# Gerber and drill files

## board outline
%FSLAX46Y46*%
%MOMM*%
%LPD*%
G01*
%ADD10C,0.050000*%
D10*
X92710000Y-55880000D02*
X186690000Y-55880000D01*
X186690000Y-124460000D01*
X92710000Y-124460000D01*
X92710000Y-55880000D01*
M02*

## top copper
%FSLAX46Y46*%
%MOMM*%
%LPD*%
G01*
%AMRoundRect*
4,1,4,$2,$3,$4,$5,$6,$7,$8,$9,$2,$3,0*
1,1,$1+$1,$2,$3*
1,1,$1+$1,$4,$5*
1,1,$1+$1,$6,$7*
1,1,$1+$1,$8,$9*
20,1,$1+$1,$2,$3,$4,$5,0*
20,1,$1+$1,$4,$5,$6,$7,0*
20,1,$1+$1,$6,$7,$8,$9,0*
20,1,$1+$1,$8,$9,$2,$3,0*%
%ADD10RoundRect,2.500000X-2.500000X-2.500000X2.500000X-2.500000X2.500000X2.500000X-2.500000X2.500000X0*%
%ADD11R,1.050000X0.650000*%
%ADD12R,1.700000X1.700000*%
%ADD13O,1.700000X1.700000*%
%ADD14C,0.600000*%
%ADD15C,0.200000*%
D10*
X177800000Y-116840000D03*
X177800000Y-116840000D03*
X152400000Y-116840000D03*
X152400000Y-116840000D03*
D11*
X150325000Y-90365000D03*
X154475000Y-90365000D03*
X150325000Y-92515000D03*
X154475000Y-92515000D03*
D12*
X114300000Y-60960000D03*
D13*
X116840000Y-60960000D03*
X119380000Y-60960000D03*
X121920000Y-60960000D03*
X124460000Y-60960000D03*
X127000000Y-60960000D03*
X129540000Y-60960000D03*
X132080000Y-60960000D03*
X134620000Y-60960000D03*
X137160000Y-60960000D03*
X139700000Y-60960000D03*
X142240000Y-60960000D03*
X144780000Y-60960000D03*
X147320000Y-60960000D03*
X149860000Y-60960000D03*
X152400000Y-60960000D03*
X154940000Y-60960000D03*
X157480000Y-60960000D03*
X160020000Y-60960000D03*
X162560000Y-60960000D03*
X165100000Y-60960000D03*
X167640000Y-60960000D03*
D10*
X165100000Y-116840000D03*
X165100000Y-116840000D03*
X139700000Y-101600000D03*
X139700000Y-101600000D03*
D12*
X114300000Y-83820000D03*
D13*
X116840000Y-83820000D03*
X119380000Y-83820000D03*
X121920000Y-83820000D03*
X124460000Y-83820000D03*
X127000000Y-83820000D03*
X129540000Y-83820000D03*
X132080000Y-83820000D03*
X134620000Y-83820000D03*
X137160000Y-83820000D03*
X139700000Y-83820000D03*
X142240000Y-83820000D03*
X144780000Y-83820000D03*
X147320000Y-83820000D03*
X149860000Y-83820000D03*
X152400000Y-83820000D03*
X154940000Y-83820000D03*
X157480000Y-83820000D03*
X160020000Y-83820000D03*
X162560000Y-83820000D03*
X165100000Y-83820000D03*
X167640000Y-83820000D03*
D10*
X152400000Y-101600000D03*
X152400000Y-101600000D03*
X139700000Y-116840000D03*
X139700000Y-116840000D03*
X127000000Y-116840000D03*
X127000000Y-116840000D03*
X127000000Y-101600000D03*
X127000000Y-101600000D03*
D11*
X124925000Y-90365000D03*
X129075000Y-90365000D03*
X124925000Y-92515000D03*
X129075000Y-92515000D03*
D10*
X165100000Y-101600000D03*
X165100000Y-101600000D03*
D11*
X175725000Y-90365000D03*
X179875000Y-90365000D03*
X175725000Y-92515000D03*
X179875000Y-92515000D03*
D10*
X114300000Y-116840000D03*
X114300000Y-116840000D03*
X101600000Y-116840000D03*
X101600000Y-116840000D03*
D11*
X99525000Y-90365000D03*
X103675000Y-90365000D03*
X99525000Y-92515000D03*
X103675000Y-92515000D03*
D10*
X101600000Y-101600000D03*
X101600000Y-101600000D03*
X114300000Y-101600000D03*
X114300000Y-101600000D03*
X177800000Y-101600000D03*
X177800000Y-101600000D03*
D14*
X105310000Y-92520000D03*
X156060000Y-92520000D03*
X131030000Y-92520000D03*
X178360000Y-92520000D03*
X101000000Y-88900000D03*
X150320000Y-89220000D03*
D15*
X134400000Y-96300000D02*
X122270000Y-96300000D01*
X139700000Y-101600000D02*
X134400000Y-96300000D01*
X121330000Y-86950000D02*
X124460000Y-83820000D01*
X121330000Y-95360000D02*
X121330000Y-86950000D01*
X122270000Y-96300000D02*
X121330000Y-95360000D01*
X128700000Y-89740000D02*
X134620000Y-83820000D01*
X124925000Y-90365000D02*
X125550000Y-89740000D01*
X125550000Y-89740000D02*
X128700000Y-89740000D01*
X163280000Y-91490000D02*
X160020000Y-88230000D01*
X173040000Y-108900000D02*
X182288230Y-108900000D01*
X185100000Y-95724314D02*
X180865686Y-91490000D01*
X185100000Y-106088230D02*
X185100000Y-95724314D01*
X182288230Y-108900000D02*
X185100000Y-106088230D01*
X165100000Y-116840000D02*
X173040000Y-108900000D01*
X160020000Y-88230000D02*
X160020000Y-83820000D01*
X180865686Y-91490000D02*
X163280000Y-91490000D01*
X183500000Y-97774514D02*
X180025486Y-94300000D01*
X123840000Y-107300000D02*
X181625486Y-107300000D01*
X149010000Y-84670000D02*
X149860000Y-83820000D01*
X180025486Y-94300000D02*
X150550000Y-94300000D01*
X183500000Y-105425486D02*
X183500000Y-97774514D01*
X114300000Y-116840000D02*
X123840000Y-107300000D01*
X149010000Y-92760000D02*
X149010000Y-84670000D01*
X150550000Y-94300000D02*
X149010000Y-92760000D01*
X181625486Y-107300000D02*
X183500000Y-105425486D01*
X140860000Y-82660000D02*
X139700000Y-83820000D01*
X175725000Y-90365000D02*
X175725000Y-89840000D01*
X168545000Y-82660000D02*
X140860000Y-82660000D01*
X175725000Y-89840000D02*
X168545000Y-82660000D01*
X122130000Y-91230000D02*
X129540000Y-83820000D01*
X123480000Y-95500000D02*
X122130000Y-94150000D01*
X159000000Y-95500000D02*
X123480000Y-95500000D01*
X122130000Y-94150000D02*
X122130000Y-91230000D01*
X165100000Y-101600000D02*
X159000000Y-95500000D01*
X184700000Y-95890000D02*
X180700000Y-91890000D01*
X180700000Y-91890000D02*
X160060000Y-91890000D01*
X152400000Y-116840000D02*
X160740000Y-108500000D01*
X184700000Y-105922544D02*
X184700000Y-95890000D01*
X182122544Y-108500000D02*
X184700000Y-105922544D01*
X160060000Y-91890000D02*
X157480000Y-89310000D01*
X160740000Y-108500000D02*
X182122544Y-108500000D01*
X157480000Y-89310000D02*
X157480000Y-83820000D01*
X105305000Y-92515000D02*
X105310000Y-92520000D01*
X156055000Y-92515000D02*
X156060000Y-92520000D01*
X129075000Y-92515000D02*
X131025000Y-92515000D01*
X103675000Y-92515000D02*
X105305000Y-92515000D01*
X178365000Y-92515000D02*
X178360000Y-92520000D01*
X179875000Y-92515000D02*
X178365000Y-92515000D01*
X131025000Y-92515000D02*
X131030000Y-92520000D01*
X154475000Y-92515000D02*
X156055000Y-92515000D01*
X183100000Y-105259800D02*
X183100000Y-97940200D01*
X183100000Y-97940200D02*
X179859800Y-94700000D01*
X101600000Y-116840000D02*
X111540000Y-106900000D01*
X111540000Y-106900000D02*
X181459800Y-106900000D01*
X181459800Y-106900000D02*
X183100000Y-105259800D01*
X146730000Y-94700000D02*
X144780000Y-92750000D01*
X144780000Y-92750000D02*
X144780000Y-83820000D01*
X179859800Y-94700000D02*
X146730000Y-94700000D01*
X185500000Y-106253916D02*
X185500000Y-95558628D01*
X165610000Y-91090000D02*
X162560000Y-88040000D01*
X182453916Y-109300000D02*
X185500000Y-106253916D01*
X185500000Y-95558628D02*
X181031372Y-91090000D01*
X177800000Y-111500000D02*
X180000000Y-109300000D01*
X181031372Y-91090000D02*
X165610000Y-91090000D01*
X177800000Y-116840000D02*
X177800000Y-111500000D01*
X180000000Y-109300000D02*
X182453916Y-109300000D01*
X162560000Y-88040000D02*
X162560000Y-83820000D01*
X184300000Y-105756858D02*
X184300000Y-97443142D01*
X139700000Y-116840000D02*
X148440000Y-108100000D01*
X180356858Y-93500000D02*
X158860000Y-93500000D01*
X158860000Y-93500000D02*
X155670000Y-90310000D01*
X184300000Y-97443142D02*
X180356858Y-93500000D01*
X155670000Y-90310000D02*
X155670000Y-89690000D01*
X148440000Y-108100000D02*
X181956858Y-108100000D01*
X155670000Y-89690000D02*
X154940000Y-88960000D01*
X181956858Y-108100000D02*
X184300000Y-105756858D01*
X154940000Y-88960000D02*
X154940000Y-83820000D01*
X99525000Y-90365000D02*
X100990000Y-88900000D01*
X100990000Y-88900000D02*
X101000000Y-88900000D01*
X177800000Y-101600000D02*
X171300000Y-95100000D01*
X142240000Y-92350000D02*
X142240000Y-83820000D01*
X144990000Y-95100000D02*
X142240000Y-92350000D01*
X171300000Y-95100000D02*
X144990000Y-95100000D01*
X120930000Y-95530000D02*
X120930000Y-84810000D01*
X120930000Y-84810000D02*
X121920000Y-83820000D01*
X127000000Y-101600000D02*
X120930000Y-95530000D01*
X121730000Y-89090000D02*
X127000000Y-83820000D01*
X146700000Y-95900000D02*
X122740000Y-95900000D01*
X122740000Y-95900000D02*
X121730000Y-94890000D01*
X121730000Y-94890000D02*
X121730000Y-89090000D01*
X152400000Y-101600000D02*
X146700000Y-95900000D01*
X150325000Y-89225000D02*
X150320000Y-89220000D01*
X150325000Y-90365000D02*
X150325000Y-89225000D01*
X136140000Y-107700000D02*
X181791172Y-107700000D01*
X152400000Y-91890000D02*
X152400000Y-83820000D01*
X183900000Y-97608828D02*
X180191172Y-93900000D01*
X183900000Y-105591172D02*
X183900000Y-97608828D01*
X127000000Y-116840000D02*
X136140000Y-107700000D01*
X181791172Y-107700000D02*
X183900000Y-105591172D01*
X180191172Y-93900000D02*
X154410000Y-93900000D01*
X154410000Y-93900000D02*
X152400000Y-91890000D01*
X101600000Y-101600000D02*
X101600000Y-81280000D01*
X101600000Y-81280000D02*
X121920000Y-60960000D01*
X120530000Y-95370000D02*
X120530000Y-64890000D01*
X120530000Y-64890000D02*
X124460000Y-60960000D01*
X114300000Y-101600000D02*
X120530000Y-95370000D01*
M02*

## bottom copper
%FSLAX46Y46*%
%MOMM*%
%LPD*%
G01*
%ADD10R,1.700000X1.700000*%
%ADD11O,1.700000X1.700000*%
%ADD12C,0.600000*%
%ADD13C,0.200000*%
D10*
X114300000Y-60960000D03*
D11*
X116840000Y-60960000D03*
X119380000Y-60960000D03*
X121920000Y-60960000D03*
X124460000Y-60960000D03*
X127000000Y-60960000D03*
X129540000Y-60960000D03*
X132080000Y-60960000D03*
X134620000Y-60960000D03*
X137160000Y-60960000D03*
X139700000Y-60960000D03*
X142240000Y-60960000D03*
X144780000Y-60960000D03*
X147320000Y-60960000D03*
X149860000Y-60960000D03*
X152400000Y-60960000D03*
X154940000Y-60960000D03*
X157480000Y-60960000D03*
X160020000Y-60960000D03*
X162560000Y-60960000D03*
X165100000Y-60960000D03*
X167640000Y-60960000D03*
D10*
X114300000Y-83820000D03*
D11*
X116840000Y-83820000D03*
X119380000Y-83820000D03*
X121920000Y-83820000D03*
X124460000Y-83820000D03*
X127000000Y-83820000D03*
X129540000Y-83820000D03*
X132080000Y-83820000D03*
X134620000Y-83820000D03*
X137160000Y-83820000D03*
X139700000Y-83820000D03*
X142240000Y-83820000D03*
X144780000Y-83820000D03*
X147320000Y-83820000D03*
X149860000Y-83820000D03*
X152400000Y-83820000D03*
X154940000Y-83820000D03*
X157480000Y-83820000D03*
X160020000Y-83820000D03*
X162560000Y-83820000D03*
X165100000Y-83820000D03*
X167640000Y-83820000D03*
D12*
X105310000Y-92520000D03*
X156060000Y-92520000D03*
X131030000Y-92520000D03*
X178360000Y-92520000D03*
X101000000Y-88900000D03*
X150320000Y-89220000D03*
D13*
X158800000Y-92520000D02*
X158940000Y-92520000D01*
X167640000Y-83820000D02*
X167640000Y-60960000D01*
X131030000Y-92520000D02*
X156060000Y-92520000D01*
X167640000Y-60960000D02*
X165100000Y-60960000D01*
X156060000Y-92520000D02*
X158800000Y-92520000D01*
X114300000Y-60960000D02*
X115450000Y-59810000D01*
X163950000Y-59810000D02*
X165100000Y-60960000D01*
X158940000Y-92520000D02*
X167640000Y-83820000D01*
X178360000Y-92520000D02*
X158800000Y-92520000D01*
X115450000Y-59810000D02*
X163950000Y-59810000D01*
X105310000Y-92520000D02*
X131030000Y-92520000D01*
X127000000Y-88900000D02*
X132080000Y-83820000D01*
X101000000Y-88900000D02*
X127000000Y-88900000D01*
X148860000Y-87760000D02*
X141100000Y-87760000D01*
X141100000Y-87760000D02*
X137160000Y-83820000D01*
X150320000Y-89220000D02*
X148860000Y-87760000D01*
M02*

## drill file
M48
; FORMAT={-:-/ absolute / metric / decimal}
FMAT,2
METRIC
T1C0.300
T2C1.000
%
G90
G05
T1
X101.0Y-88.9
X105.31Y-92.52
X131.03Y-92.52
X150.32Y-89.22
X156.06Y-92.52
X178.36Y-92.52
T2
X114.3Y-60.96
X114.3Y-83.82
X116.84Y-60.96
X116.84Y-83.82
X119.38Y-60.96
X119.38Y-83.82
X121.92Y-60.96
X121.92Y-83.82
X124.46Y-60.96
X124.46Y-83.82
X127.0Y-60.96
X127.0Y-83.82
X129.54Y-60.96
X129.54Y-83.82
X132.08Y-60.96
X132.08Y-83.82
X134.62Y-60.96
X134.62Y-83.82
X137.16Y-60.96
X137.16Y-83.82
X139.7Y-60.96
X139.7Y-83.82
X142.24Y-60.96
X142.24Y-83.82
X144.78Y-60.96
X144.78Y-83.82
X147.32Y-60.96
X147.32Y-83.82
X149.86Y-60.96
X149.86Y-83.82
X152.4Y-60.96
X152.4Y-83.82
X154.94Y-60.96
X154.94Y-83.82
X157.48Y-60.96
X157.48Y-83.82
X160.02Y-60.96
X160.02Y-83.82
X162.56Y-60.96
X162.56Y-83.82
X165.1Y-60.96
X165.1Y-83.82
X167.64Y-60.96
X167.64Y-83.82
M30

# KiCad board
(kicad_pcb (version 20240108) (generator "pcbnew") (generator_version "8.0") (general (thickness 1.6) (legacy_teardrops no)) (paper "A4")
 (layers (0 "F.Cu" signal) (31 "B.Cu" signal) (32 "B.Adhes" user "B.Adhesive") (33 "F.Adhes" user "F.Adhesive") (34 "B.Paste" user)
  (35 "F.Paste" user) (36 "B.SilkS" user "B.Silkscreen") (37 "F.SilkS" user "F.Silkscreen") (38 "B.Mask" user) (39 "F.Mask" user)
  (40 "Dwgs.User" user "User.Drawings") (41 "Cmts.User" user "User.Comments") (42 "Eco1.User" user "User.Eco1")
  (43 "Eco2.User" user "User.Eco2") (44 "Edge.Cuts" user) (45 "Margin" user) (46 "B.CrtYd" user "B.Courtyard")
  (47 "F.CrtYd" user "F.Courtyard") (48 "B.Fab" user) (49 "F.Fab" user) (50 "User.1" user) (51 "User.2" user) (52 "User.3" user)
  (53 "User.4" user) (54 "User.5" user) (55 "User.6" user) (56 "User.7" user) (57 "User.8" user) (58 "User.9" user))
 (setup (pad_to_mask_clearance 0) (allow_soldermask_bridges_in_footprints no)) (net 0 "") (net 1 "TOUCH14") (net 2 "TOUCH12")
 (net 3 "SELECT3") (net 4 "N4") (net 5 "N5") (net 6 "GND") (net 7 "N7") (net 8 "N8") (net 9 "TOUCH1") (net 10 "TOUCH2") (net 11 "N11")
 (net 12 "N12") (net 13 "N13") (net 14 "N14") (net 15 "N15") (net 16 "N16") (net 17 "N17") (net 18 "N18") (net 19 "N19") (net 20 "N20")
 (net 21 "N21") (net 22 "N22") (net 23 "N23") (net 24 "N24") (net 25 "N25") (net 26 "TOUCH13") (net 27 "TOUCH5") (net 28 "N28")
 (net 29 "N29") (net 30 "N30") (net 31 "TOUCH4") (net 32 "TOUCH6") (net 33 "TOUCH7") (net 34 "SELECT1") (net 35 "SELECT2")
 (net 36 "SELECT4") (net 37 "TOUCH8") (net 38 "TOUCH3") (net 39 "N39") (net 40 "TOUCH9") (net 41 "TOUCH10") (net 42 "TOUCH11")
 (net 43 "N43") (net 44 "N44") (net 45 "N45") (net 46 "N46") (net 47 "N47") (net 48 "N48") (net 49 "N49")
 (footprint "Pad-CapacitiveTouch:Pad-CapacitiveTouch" (layer "F.Cu") (at 177.8 116.84)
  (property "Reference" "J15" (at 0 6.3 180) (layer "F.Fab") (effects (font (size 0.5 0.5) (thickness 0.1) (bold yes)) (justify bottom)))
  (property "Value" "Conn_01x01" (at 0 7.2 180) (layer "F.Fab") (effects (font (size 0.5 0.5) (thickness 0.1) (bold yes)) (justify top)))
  (pad "1" smd roundrect (at 0 0) (size 10 10) (layers "F.Cu") (roundrect_rratio 0.25) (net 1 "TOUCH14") (thermal_bridge_angle 0))
  (pad "1" smd roundrect (at 0 0) (size 10 10) (layers "F.Cu" "F.Mask") (roundrect_rratio 0.25) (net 1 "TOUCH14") (thermal_bridge_angle 0)))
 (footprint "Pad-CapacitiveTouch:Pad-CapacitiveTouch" (layer "F.Cu") (at 152.4 116.84)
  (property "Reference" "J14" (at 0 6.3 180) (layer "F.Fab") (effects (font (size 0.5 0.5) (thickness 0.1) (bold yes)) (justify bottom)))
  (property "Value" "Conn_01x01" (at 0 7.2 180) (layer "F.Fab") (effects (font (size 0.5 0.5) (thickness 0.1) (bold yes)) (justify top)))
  (pad "1" smd roundrect (at 0 0) (size 10 10) (layers "F.Cu") (roundrect_rratio 0.25) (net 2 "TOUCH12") (thermal_bridge_angle 0))
  (pad "1" smd roundrect (at 0 0) (size 10 10) (layers "F.Cu" "F.Mask") (roundrect_rratio 0.25) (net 2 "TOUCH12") (thermal_bridge_angle 0)))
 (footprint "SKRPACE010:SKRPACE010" (layer "F.Cu") (at 152.4 91.44)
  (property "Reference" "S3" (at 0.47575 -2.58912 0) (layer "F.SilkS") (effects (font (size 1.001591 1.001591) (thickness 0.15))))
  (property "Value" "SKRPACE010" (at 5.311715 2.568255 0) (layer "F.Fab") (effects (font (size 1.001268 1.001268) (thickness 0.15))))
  (pad "1" smd rect (at -2.075 -1.075) (size 1.05 0.65) (layers "F.Cu" "F.Paste" "F.Mask") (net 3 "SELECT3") (solder_mask_margin 0.102))
  (pad "2" smd rect (at 2.075 -1.075) (size 1.05 0.65) (layers "F.Cu" "F.Paste" "F.Mask") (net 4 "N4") (solder_mask_margin 0.102))
  (pad "3" smd rect (at -2.075 1.075) (size 1.05 0.65) (layers "F.Cu" "F.Paste" "F.Mask") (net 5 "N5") (solder_mask_margin 0.102))
  (pad "4" smd rect (at 2.075 1.075) (size 1.05 0.65) (layers "F.Cu" "F.Paste" "F.Mask") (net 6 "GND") (solder_mask_margin 0.102)))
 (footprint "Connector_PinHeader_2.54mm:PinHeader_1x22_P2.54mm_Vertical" (layer "F.Cu") (at 114.3 60.96 90)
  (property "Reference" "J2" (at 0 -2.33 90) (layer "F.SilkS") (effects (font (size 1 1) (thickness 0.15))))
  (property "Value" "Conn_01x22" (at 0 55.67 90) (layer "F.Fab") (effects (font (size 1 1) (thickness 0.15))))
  (pad "1" thru_hole rect (at 0 0 90) (size 1.7 1.7) (drill 1) (layers "*.Cu" "*.Mask") (remove_unused_layers no) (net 6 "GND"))
  (pad "2" thru_hole oval (at 0 2.54 90) (size 1.7 1.7) (drill 1) (layers "*.Cu" "*.Mask") (remove_unused_layers no) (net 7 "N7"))
  (pad "3" thru_hole oval (at 0 5.08 90) (size 1.7 1.7) (drill 1) (layers "*.Cu" "*.Mask") (remove_unused_layers no) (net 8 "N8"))
  (pad "4" thru_hole oval (at 0 7.62 90) (size 1.7 1.7) (drill 1) (layers "*.Cu" "*.Mask") (remove_unused_layers no) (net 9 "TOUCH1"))
  (pad "5" thru_hole oval (at 0 10.16 90) (size 1.7 1.7) (drill 1) (layers "*.Cu" "*.Mask") (remove_unused_layers no) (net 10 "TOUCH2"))
  (pad "6" thru_hole oval (at 0 12.7 90) (size 1.7 1.7) (drill 1) (layers "*.Cu" "*.Mask") (remove_unused_layers no) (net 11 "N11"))
  (pad "7" thru_hole oval (at 0 15.24 90) (size 1.7 1.7) (drill 1) (layers "*.Cu" "*.Mask") (remove_unused_layers no) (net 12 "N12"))
  (pad "8" thru_hole oval (at 0 17.78 90) (size 1.7 1.7) (drill 1) (layers "*.Cu" "*.Mask") (remove_unused_layers no) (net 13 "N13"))
  (pad "9" thru_hole oval (at 0 20.32 90) (size 1.7 1.7) (drill 1) (layers "*.Cu" "*.Mask") (remove_unused_layers no) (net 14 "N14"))
  (pad "10" thru_hole oval (at 0 22.86 90) (size 1.7 1.7) (drill 1) (layers "*.Cu" "*.Mask") (remove_unused_layers no) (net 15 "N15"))
  (pad "11" thru_hole oval (at 0 25.4 90) (size 1.7 1.7) (drill 1) (layers "*.Cu" "*.Mask") (remove_unused_layers no) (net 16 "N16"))
  (pad "12" thru_hole oval (at 0 27.94 90) (size 1.7 1.7) (drill 1) (layers "*.Cu" "*.Mask") (remove_unused_layers no) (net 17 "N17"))
  (pad "13" thru_hole oval (at 0 30.48 90) (size 1.7 1.7) (drill 1) (layers "*.Cu" "*.Mask") (remove_unused_layers no) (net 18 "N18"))
  (pad "14" thru_hole oval (at 0 33.02 90) (size 1.7 1.7) (drill 1) (layers "*.Cu" "*.Mask") (remove_unused_layers no) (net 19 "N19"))
  (pad "15" thru_hole oval (at 0 35.56 90) (size 1.7 1.7) (drill 1) (layers "*.Cu" "*.Mask") (remove_unused_layers no) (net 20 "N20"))
  (pad "16" thru_hole oval (at 0 38.1 90) (size 1.7 1.7) (drill 1) (layers "*.Cu" "*.Mask") (remove_unused_layers no) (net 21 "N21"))
  (pad "17" thru_hole oval (at 0 40.64 90) (size 1.7 1.7) (drill 1) (layers "*.Cu" "*.Mask") (remove_unused_layers no) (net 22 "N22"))
  (pad "18" thru_hole oval (at 0 43.18 90) (size 1.7 1.7) (drill 1) (layers "*.Cu" "*.Mask") (remove_unused_layers no) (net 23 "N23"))
  (pad "19" thru_hole oval (at 0 45.72 90) (size 1.7 1.7) (drill 1) (layers "*.Cu" "*.Mask") (remove_unused_layers no) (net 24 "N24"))
  (pad "20" thru_hole oval (at 0 48.26 90) (size 1.7 1.7) (drill 1) (layers "*.Cu" "*.Mask") (remove_unused_layers no) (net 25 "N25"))
  (pad "21" thru_hole oval (at 0 50.8 90) (size 1.7 1.7) (drill 1) (layers "*.Cu" "*.Mask") (remove_unused_layers no) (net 6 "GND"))
  (pad "22" thru_hole oval (at 0 53.34 90) (size 1.7 1.7) (drill 1) (layers "*.Cu" "*.Mask") (remove_unused_layers no) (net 6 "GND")))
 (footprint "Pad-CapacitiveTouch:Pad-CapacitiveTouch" (layer "F.Cu") (at 165.1 116.84)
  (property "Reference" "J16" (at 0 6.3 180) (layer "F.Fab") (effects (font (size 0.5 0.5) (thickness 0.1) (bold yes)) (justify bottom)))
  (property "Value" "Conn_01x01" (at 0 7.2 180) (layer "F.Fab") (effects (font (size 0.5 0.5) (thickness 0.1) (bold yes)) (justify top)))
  (pad "1" smd roundrect (at 0 0) (size 10 10) (layers "F.Cu") (roundrect_rratio 0.25) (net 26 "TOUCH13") (thermal_bridge_angle 0))
  (pad "1" smd roundrect (at 0 0) (size 10 10) (layers "F.Cu" "F.Mask") (roundrect_rratio 0.25) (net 26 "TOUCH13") (thermal_bridge_angle 0)))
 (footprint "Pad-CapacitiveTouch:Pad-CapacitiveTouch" (layer "F.Cu") (at 139.7 101.6)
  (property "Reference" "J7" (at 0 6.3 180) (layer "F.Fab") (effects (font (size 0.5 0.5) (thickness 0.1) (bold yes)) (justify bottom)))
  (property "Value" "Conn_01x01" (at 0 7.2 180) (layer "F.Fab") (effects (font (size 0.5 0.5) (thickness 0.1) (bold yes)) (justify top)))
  (pad "1" smd roundrect (at 0 0) (size 10 10) (layers "F.Cu") (roundrect_rratio 0.25) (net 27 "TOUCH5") (thermal_bridge_angle 0))
  (pad "1" smd roundrect (at 0 0) (size 10 10) (layers "F.Cu" "F.Mask") (roundrect_rratio 0.25) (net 27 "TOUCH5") (thermal_bridge_angle 0)))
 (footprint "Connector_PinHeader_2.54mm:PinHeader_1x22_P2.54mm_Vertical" (layer "F.Cu") (at 114.3 83.82 90)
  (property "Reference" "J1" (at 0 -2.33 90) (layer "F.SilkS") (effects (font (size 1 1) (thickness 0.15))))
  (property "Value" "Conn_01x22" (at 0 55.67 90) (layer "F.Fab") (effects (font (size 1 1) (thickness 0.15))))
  (pad "1" thru_hole rect (at 0 0 90) (size 1.7 1.7) (drill 1) (layers "*.Cu" "*.Mask") (remove_unused_layers no) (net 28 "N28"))
  (pad "2" thru_hole oval (at 0 2.54 90) (size 1.7 1.7) (drill 1) (layers "*.Cu" "*.Mask") (remove_unused_layers no) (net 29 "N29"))
  (pad "3" thru_hole oval (at 0 5.08 90) (size 1.7 1.7) (drill 1) (layers "*.Cu" "*.Mask") (remove_unused_layers no) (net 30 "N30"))
  (pad "4" thru_hole oval (at 0 7.62 90) (size 1.7 1.7) (drill 1) (layers "*.Cu" "*.Mask") (remove_unused_layers no) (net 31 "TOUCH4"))
  (pad "5" thru_hole oval (at 0 10.16 90) (size 1.7 1.7) (drill 1) (layers "*.Cu" "*.Mask") (remove_unused_layers no) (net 27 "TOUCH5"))
  (pad "6" thru_hole oval (at 0 12.7 90) (size 1.7 1.7) (drill 1) (layers "*.Cu" "*.Mask") (remove_unused_layers no) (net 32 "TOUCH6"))
  (pad "7" thru_hole oval (at 0 15.24 90) (size 1.7 1.7) (drill 1) (layers "*.Cu" "*.Mask") (remove_unused_layers no) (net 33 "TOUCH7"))
  (pad "8" thru_hole oval (at 0 17.78 90) (size 1.7 1.7) (drill 1) (layers "*.Cu" "*.Mask") (remove_unused_layers no) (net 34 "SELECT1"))
  (pad "9" thru_hole oval (at 0 20.32 90) (size 1.7 1.7) (drill 1) (layers "*.Cu" "*.Mask") (remove_unused_layers no) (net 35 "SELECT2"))
  (pad "10" thru_hole oval (at 0 22.86 90) (size 1.7 1.7) (drill 1) (layers "*.Cu" "*.Mask") (remove_unused_layers no) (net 3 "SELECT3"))
  (pad "11" thru_hole oval (at 0 25.4 90) (size 1.7 1.7) (drill 1) (layers "*.Cu" "*.Mask") (remove_unused_layers no) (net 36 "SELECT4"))
  (pad "12" thru_hole oval (at 0 27.94 90) (size 1.7 1.7) (drill 1) (layers "*.Cu" "*.Mask") (remove_unused_layers no) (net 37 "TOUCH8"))
  (pad "13" thru_hole oval (at 0 30.48 90) (size 1.7 1.7) (drill 1) (layers "*.Cu" "*.Mask") (remove_unused_layers no) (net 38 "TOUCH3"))
  (pad "14" thru_hole oval (at 0 33.02 90) (size 1.7 1.7) (drill 1) (layers "*.Cu" "*.Mask") (remove_unused_layers no) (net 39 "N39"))
  (pad "15" thru_hole oval (at 0 35.56 90) (size 1.7 1.7) (drill 1) (layers "*.Cu" "*.Mask") (remove_unused_layers no) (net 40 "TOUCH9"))
  (pad "16" thru_hole oval (at 0 38.1 90) (size 1.7 1.7) (drill 1) (layers "*.Cu" "*.Mask") (remove_unused_layers no) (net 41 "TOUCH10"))
  (pad "17" thru_hole oval (at 0 40.64 90) (size 1.7 1.7) (drill 1) (layers "*.Cu" "*.Mask") (remove_unused_layers no) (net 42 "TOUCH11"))
  (pad "18" thru_hole oval (at 0 43.18 90) (size 1.7 1.7) (drill 1) (layers "*.Cu" "*.Mask") (remove_unused_layers no) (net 2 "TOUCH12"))
  (pad "19" thru_hole oval (at 0 45.72 90) (size 1.7 1.7) (drill 1) (layers "*.Cu" "*.Mask") (remove_unused_layers no) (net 26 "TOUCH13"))
  (pad "20" thru_hole oval (at 0 48.26 90) (size 1.7 1.7) (drill 1) (layers "*.Cu" "*.Mask") (remove_unused_layers no) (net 1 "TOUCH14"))
  (pad "21" thru_hole oval (at 0 50.8 90) (size 1.7 1.7) (drill 1) (layers "*.Cu" "*.Mask") (remove_unused_layers no) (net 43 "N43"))
  (pad "22" thru_hole oval (at 0 53.34 90) (size 1.7 1.7) (drill 1) (layers "*.Cu" "*.Mask") (remove_unused_layers no) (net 6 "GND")))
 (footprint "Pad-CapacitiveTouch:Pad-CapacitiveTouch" (layer "F.Cu") (at 152.4 101.6)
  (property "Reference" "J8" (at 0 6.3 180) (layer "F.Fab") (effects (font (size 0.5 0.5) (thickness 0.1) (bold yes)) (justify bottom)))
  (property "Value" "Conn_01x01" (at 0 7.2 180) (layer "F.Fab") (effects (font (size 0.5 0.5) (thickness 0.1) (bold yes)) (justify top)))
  (pad "1" smd roundrect (at 0 0) (size 10 10) (layers "F.Cu") (roundrect_rratio 0.25) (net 32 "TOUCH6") (thermal_bridge_angle 0))
  (pad "1" smd roundrect (at 0 0) (size 10 10) (layers "F.Cu" "F.Mask") (roundrect_rratio 0.25) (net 32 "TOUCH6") (thermal_bridge_angle 0)))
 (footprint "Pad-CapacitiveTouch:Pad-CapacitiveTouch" (layer "F.Cu") (at 139.7 116.84)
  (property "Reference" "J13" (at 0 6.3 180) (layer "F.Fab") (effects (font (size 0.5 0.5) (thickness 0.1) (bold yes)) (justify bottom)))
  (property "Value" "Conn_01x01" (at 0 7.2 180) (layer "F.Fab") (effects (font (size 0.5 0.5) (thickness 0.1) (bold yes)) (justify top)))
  (pad "1" smd roundrect (at 0 0) (size 10 10) (layers "F.Cu") (roundrect_rratio 0.25) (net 42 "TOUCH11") (thermal_bridge_angle 0))
  (pad "1" smd roundrect (at 0 0) (size 10 10) (layers "F.Cu" "F.Mask") (roundrect_rratio 0.25) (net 42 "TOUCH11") (thermal_bridge_angle 0)))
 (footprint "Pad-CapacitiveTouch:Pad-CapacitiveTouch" (layer "F.Cu") (at 127 116.84)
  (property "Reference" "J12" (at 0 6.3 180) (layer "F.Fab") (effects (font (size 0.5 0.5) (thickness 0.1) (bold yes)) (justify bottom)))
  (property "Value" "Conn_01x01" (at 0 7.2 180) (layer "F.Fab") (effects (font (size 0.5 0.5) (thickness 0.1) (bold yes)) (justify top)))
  (pad "1" smd roundrect (at 0 0) (size 10 10) (layers "F.Cu") (roundrect_rratio 0.25) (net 41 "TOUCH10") (thermal_bridge_angle 0))
  (pad "1" smd roundrect (at 0 0) (size 10 10) (layers "F.Cu" "F.Mask") (roundrect_rratio 0.25) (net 41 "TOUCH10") (thermal_bridge_angle 0)))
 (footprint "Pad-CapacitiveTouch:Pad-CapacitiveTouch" (layer "F.Cu") (at 127 101.6)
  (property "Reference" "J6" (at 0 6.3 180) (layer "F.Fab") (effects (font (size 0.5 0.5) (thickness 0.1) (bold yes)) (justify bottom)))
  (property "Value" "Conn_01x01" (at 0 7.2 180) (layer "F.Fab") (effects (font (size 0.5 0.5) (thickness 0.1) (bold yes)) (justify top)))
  (pad "1" smd roundrect (at 0 0) (size 10 10) (layers "F.Cu") (roundrect_rratio 0.25) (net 31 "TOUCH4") (thermal_bridge_angle 0))
  (pad "1" smd roundrect (at 0 0) (size 10 10) (layers "F.Cu" "F.Mask") (roundrect_rratio 0.25) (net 31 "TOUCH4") (thermal_bridge_angle 0)))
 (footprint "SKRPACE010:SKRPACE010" (layer "F.Cu") (at 127 91.44)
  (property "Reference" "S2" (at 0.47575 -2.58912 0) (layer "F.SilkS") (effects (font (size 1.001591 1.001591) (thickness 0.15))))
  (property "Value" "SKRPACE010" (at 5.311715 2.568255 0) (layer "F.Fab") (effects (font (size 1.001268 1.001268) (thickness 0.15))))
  (pad "1" smd rect (at -2.075 -1.075) (size 1.05 0.65) (layers "F.Cu" "F.Paste" "F.Mask") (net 35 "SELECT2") (solder_mask_margin 0.102))
  (pad "2" smd rect (at 2.075 -1.075) (size 1.05 0.65) (layers "F.Cu" "F.Paste" "F.Mask") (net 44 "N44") (solder_mask_margin 0.102))
  (pad "3" smd rect (at -2.075 1.075) (size 1.05 0.65) (layers "F.Cu" "F.Paste" "F.Mask") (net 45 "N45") (solder_mask_margin 0.102))
  (pad "4" smd rect (at 2.075 1.075) (size 1.05 0.65) (layers "F.Cu" "F.Paste" "F.Mask") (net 6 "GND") (solder_mask_margin 0.102)))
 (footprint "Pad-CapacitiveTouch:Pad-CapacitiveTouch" (layer "F.Cu") (at 165.1 101.6)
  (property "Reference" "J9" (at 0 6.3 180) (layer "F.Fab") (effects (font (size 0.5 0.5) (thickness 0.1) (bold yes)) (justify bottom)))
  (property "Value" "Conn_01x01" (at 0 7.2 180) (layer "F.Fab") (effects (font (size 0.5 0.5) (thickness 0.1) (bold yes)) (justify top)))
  (pad "1" smd roundrect (at 0 0) (size 10 10) (layers "F.Cu") (roundrect_rratio 0.25) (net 33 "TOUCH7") (thermal_bridge_angle 0))
  (pad "1" smd roundrect (at 0 0) (size 10 10) (layers "F.Cu" "F.Mask") (roundrect_rratio 0.25) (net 33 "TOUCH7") (thermal_bridge_angle 0)))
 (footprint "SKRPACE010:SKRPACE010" (layer "F.Cu") (at 177.8 91.44)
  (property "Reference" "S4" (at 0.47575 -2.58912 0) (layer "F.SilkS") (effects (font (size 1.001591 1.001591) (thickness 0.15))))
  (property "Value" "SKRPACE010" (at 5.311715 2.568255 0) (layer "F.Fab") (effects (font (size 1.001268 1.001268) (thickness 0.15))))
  (pad "1" smd rect (at -2.075 -1.075) (size 1.05 0.65) (layers "F.Cu" "F.Paste" "F.Mask") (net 36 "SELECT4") (solder_mask_margin 0.102))
  (pad "2" smd rect (at 2.075 -1.075) (size 1.05 0.65) (layers "F.Cu" "F.Paste" "F.Mask") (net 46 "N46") (solder_mask_margin 0.102))
  (pad "3" smd rect (at -2.075 1.075) (size 1.05 0.65) (layers "F.Cu" "F.Paste" "F.Mask") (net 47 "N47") (solder_mask_margin 0.102))
  (pad "4" smd rect (at 2.075 1.075) (size 1.05 0.65) (layers "F.Cu" "F.Paste" "F.Mask") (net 6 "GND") (solder_mask_margin 0.102)))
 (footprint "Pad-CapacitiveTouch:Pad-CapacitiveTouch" (layer "F.Cu") (at 114.3 116.84)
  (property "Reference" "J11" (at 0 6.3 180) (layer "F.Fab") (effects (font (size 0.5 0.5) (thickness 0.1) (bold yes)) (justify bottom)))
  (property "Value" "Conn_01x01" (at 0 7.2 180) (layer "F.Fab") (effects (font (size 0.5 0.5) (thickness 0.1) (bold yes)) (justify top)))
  (pad "1" smd roundrect (at 0 0) (size 10 10) (layers "F.Cu") (roundrect_rratio 0.25) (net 40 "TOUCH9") (thermal_bridge_angle 0))
  (pad "1" smd roundrect (at 0 0) (size 10 10) (layers "F.Cu" "F.Mask") (roundrect_rratio 0.25) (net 40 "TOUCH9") (thermal_bridge_angle 0)))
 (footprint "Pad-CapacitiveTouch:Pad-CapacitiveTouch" (layer "F.Cu") (at 101.6 116.84)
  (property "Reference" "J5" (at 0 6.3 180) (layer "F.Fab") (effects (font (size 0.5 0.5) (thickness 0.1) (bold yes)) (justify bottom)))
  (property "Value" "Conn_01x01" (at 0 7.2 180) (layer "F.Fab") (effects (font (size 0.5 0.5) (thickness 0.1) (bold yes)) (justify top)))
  (pad "1" smd roundrect (at 0 0) (size 10 10) (layers "F.Cu") (roundrect_rratio 0.25) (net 38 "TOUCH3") (thermal_bridge_angle 0))
  (pad "1" smd roundrect (at 0 0) (size 10 10) (layers "F.Cu" "F.Mask") (roundrect_rratio 0.25) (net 38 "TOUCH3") (thermal_bridge_angle 0)))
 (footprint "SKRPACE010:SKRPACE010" (layer "F.Cu") (at 101.6 91.44)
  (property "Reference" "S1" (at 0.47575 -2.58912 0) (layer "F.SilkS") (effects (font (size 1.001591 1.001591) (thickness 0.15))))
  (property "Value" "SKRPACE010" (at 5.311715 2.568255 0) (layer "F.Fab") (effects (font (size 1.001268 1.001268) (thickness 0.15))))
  (pad "1" smd rect (at -2.075 -1.075) (size 1.05 0.65) (layers "F.Cu" "F.Paste" "F.Mask") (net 34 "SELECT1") (solder_mask_margin 0.102))
  (pad "2" smd rect (at 2.075 -1.075) (size 1.05 0.65) (layers "F.Cu" "F.Paste" "F.Mask") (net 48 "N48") (solder_mask_margin 0.102))
  (pad "3" smd rect (at -2.075 1.075) (size 1.05 0.65) (layers "F.Cu" "F.Paste" "F.Mask") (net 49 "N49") (solder_mask_margin 0.102))
  (pad "4" smd rect (at 2.075 1.075) (size 1.05 0.65) (layers "F.Cu" "F.Paste" "F.Mask") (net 6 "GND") (solder_mask_margin 0.102)))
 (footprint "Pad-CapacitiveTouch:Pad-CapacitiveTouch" (layer "F.Cu") (at 101.6 101.6)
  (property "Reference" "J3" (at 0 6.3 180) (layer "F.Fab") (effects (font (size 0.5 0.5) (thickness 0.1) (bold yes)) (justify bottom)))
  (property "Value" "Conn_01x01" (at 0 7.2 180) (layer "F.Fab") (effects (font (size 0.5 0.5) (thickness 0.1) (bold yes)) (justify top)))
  (pad "1" smd roundrect (at 0 0) (size 10 10) (layers "F.Cu") (roundrect_rratio 0.25) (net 9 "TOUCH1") (thermal_bridge_angle 0))
  (pad "1" smd roundrect (at 0 0) (size 10 10) (layers "F.Cu" "F.Mask") (roundrect_rratio 0.25) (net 9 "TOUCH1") (thermal_bridge_angle 0)))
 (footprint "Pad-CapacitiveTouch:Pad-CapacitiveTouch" (layer "F.Cu") (at 114.3 101.6)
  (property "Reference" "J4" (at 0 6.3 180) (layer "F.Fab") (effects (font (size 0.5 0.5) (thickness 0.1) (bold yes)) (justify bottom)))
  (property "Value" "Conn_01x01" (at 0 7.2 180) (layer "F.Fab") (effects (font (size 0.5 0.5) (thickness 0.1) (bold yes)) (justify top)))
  (pad "1" smd roundrect (at 0 0) (size 10 10) (layers "F.Cu") (roundrect_rratio 0.25) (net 10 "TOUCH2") (thermal_bridge_angle 0))
  (pad "1" smd roundrect (at 0 0) (size 10 10) (layers "F.Cu" "F.Mask") (roundrect_rratio 0.25) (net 10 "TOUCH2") (thermal_bridge_angle 0)))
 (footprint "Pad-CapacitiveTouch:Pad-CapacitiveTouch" (layer "F.Cu") (at 177.8 101.6)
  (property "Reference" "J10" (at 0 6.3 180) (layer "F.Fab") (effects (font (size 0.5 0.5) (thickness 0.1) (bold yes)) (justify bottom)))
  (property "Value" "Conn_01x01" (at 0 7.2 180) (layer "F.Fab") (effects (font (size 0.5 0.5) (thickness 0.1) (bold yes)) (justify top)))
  (pad "1" smd roundrect (at 0 0) (size 10 10) (layers "F.Cu") (roundrect_rratio 0.25) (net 37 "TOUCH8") (thermal_bridge_angle 0))
  (pad "1" smd roundrect (at 0 0) (size 10 10) (layers "F.Cu" "F.Mask") (roundrect_rratio 0.25) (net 37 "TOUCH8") (thermal_bridge_angle 0)))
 (gr_rect (start 92.71 55.88) (end 186.69 124.46) (stroke (width 0.05) (type default)) (fill none) (layer "Edge.Cuts"))
 (segment (start 134.4 96.3) (end 122.27 96.3) (width 0.2) (layer "F.Cu") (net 27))
 (segment (start 139.7 101.6) (end 134.4 96.3) (width 0.2) (layer "F.Cu") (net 27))
 (segment (start 121.33 86.95) (end 124.46 83.82) (width 0.2) (layer "F.Cu") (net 27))
 (segment (start 121.33 95.36) (end 121.33 86.95) (width 0.2) (layer "F.Cu") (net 27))
 (segment (start 122.27 96.3) (end 121.33 95.36) (width 0.2) (layer "F.Cu") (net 27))
 (segment (start 128.7 89.74) (end 134.62 83.82) (width 0.2) (layer "F.Cu") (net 35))
 (segment (start 124.925 90.365) (end 125.55 89.74) (width 0.2) (layer "F.Cu") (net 35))
 (segment (start 125.55 89.74) (end 128.7 89.74) (width 0.2) (layer "F.Cu") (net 35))
 (segment (start 163.28 91.49) (end 160.02 88.23) (width 0.2) (layer "F.Cu") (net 26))
 (segment (start 173.04 108.9) (end 182.28823 108.9) (width 0.2) (layer "F.Cu") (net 26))
 (segment (start 185.1 95.724314) (end 180.865686 91.49) (width 0.2) (layer "F.Cu") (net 26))
 (segment (start 185.1 106.08823) (end 185.1 95.724314) (width 0.2) (layer "F.Cu") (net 26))
 (segment (start 182.28823 108.9) (end 185.1 106.08823) (width 0.2) (layer "F.Cu") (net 26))
 (segment (start 165.1 116.84) (end 173.04 108.9) (width 0.2) (layer "F.Cu") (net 26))
 (segment (start 160.02 88.23) (end 160.02 83.82) (width 0.2) (layer "F.Cu") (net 26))
 (segment (start 180.865686 91.49) (end 163.28 91.49) (width 0.2) (layer "F.Cu") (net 26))
 (segment (start 183.5 97.774514) (end 180.025486 94.3) (width 0.2) (layer "F.Cu") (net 40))
 (segment (start 123.84 107.3) (end 181.625486 107.3) (width 0.2) (layer "F.Cu") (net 40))
 (segment (start 149.01 84.67) (end 149.86 83.82) (width 0.2) (layer "F.Cu") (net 40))
 (segment (start 180.025486 94.3) (end 150.55 94.3) (width 0.2) (layer "F.Cu") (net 40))
 (segment (start 183.5 105.425486) (end 183.5 97.774514) (width 0.2) (layer "F.Cu") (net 40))
 (segment (start 114.3 116.84) (end 123.84 107.3) (width 0.2) (layer "F.Cu") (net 40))
 (segment (start 149.01 92.76) (end 149.01 84.67) (width 0.2) (layer "F.Cu") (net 40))
 (segment (start 150.55 94.3) (end 149.01 92.76) (width 0.2) (layer "F.Cu") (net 40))
 (segment (start 181.625486 107.3) (end 183.5 105.425486) (width 0.2) (layer "F.Cu") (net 40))
 (segment (start 140.86 82.66) (end 139.7 83.82) (width 0.2) (layer "F.Cu") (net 36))
 (segment (start 175.725 90.365) (end 175.725 89.84) (width 0.2) (layer "F.Cu") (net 36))
 (segment (start 168.545 82.66) (end 140.86 82.66) (width 0.2) (layer "F.Cu") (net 36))
 (segment (start 175.725 89.84) (end 168.545 82.66) (width 0.2) (layer "F.Cu") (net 36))
 (segment (start 122.13 91.23) (end 129.54 83.82) (width 0.2) (layer "F.Cu") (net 33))
 (segment (start 123.48 95.5) (end 122.13 94.15) (width 0.2) (layer "F.Cu") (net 33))
 (segment (start 159 95.5) (end 123.48 95.5) (width 0.2) (layer "F.Cu") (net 33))
 (segment (start 122.13 94.15) (end 122.13 91.23) (width 0.2) (layer "F.Cu") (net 33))
 (segment (start 165.1 101.6) (end 159 95.5) (width 0.2) (layer "F.Cu") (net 33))
 (segment (start 184.7 95.89) (end 180.7 91.89) (width 0.2) (layer "F.Cu") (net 2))
 (segment (start 180.7 91.89) (end 160.06 91.89) (width 0.2) (layer "F.Cu") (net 2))
 (segment (start 152.4 116.84) (end 160.74 108.5) (width 0.2) (layer "F.Cu") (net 2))
 (segment (start 184.7 105.922544) (end 184.7 95.89) (width 0.2) (layer "F.Cu") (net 2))
 (segment (start 182.122544 108.5) (end 184.7 105.922544) (width 0.2) (layer "F.Cu") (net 2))
 (segment (start 160.06 91.89) (end 157.48 89.31) (width 0.2) (layer "F.Cu") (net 2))
 (segment (start 160.74 108.5) (end 182.122544 108.5) (width 0.2) (layer "F.Cu") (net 2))
 (segment (start 157.48 89.31) (end 157.48 83.82) (width 0.2) (layer "F.Cu") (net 2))
 (segment (start 105.305 92.515) (end 105.31 92.52) (width 0.2) (layer "F.Cu") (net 6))
 (segment (start 156.055 92.515) (end 156.06 92.52) (width 0.2) (layer "F.Cu") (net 6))
 (segment (start 129.075 92.515) (end 131.025 92.515) (width 0.2) (layer "F.Cu") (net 6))
 (segment (start 103.675 92.515) (end 105.305 92.515) (width 0.2) (layer "F.Cu") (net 6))
 (segment (start 178.365 92.515) (end 178.36 92.52) (width 0.2) (layer "F.Cu") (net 6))
 (segment (start 179.875 92.515) (end 178.365 92.515) (width 0.2) (layer "F.Cu") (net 6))
 (segment (start 131.025 92.515) (end 131.03 92.52) (width 0.2) (layer "F.Cu") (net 6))
 (segment (start 154.475 92.515) (end 156.055 92.515) (width 0.2) (layer "F.Cu") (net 6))
 (via (at 105.31 92.52) (size 0.6) (drill 0.3) (layers "F.Cu" "B.Cu") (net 6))
 (via (at 156.06 92.52) (size 0.6) (drill 0.3) (layers "F.Cu" "B.Cu") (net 6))
 (via (at 131.03 92.52) (size 0.6) (drill 0.3) (layers "F.Cu" "B.Cu") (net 6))
 (via (at 178.36 92.52) (size 0.6) (drill 0.3) (layers "F.Cu" "B.Cu") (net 6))
 (segment (start 158.8 92.52) (end 158.94 92.52) (width 0.2) (layer "B.Cu") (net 6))
 (segment (start 167.64 83.82) (end 167.64 60.96) (width 0.2) (layer "B.Cu") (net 6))
 (segment (start 131.03 92.52) (end 156.06 92.52) (width 0.2) (layer "B.Cu") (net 6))
 (segment (start 167.64 60.96) (end 165.1 60.96) (width 0.2) (layer "B.Cu") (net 6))
 (segment (start 156.06 92.52) (end 158.8 92.52) (width 0.2) (layer "B.Cu") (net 6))
 (segment (start 114.3 60.96) (end 115.45 59.81) (width 0.2) (layer "B.Cu") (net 6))
 (segment (start 163.95 59.81) (end 165.1 60.96) (width 0.2) (layer "B.Cu") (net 6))
 (segment (start 158.94 92.52) (end 167.64 83.82) (width 0.2) (layer "B.Cu") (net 6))
 (segment (start 178.36 92.52) (end 158.8 92.52) (width 0.2) (layer "B.Cu") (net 6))
 (segment (start 115.45 59.81) (end 163.95 59.81) (width 0.2) (layer "B.Cu") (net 6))
 (segment (start 105.31 92.52) (end 131.03 92.52) (width 0.2) (layer "B.Cu") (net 6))
 (segment (start 183.1 105.2598) (end 183.1 97.9402) (width 0.2) (layer "F.Cu") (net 38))
 (segment (start 183.1 97.9402) (end 179.8598 94.7) (width 0.2) (layer "F.Cu") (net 38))
 (segment (start 101.6 116.84) (end 111.54 106.9) (width 0.2) (layer "F.Cu") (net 38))
 (segment (start 111.54 106.9) (end 181.4598 106.9) (width 0.2) (layer "F.Cu") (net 38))
 (segment (start 181.4598 106.9) (end 183.1 105.2598) (width 0.2) (layer "F.Cu") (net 38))
 (segment (start 146.73 94.7) (end 144.78 92.75) (width 0.2) (layer "F.Cu") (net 38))
 (segment (start 144.78 92.75) (end 144.78 83.82) (width 0.2) (layer "F.Cu") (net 38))
 (segment (start 179.8598 94.7) (end 146.73 94.7) (width 0.2) (layer "F.Cu") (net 38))
 (segment (start 185.5 106.253916) (end 185.5 95.558628) (width 0.2) (layer "F.Cu") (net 1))
 (segment (start 165.61 91.09) (end 162.56 88.04) (width 0.2) (layer "F.Cu") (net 1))
 (segment (start 182.453916 109.3) (end 185.5 106.253916) (width 0.2) (layer "F.Cu") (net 1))
 (segment (start 185.5 95.558628) (end 181.031372 91.09) (width 0.2) (layer "F.Cu") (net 1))
 (segment (start 177.8 111.5) (end 180 109.3) (width 0.2) (layer "F.Cu") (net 1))
 (segment (start 181.031372 91.09) (end 165.61 91.09) (width 0.2) (layer "F.Cu") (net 1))
 (segment (start 177.8 116.84) (end 177.8 111.5) (width 0.2) (layer "F.Cu") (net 1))
 (segment (start 180 109.3) (end 182.453916 109.3) (width 0.2) (layer "F.Cu") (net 1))
 (segment (start 162.56 88.04) (end 162.56 83.82) (width 0.2) (layer "F.Cu") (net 1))
 (segment (start 184.3 105.756858) (end 184.3 97.443142) (width 0.2) (layer "F.Cu") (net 42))
 (segment (start 139.7 116.84) (end 148.44 108.1) (width 0.2) (layer "F.Cu") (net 42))
 (segment (start 180.356858 93.5) (end 158.86 93.5) (width 0.2) (layer "F.Cu") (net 42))
 (segment (start 158.86 93.5) (end 155.67 90.31) (width 0.2) (layer "F.Cu") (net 42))
 (segment (start 184.3 97.443142) (end 180.356858 93.5) (width 0.2) (layer "F.Cu") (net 42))
 (segment (start 155.67 90.31) (end 155.67 89.69) (width 0.2) (layer "F.Cu") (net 42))
 (segment (start 148.44 108.1) (end 181.956858 108.1) (width 0.2) (layer "F.Cu") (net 42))
 (segment (start 155.67 89.69) (end 154.94 88.96) (width 0.2) (layer "F.Cu") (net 42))
 (segment (start 181.956858 108.1) (end 184.3 105.756858) (width 0.2) (layer "F.Cu") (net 42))
 (segment (start 154.94 88.96) (end 154.94 83.82) (width 0.2) (layer "F.Cu") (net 42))
 (segment (start 99.525 90.365) (end 100.99 88.9) (width 0.2) (layer "F.Cu") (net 34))
 (segment (start 100.99 88.9) (end 101 88.9) (width 0.2) (layer "F.Cu") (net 34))
 (via (at 101 88.9) (size 0.6) (drill 0.3) (layers "F.Cu" "B.Cu") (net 34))
 (segment (start 127 88.9) (end 132.08 83.82) (width 0.2) (layer "B.Cu") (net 34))
 (segment (start 101 88.9) (end 127 88.9) (width 0.2) (layer "B.Cu") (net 34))
 (segment (start 177.8 101.6) (end 171.3 95.1) (width 0.2) (layer "F.Cu") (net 37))
 (segment (start 142.24 92.35) (end 142.24 83.82) (width 0.2) (layer "F.Cu") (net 37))
 (segment (start 144.99 95.1) (end 142.24 92.35) (width 0.2) (layer "F.Cu") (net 37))
 (segment (start 171.3 95.1) (end 144.99 95.1) (width 0.2) (layer "F.Cu") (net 37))
 (segment (start 120.93 95.53) (end 120.93 84.81) (width 0.2) (layer "F.Cu") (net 31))
 (segment (start 120.93 84.81) (end 121.92 83.82) (width 0.2) (layer "F.Cu") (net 31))
 (segment (start 127 101.6) (end 120.93 95.53) (width 0.2) (layer "F.Cu") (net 31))
 (segment (start 121.73 89.09) (end 127 83.82) (width 0.2) (layer "F.Cu") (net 32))
 (segment (start 146.7 95.9) (end 122.74 95.9) (width 0.2) (layer "F.Cu") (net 32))
 (segment (start 122.74 95.9) (end 121.73 94.89) (width 0.2) (layer "F.Cu") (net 32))
 (segment (start 121.73 94.89) (end 121.73 89.09) (width 0.2) (layer "F.Cu") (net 32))
 (segment (start 152.4 101.6) (end 146.7 95.9) (width 0.2) (layer "F.Cu") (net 32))
 (segment (start 150.325 89.225) (end 150.32 89.22) (width 0.2) (layer "F.Cu") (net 3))
 (segment (start 150.325 90.365) (end 150.325 89.225) (width 0.2) (layer "F.Cu") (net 3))
 (via (at 150.32 89.22) (size 0.6) (drill 0.3) (layers "F.Cu" "B.Cu") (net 3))
 (segment (start 148.86 87.76) (end 141.1 87.76) (width 0.2) (layer "B.Cu") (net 3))
 (segment (start 141.1 87.76) (end 137.16 83.82) (width 0.2) (layer "B.Cu") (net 3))
 (segment (start 150.32 89.22) (end 148.86 87.76) (width 0.2) (layer "B.Cu") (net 3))
 (segment (start 136.14 107.7) (end 181.791172 107.7) (width 0.2) (layer "F.Cu") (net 41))
 (segment (start 152.4 91.89) (end 152.4 83.82) (width 0.2) (layer "F.Cu") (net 41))
 (segment (start 183.9 97.608828) (end 180.191172 93.9) (width 0.2) (layer "F.Cu") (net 41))
 (segment (start 183.9 105.591172) (end 183.9 97.608828) (width 0.2) (layer "F.Cu") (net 41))
 (segment (start 127 116.84) (end 136.14 107.7) (width 0.2) (layer "F.Cu") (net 41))
 (segment (start 181.791172 107.7) (end 183.9 105.591172) (width 0.2) (layer "F.Cu") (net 41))
 (segment (start 180.191172 93.9) (end 154.41 93.9) (width 0.2) (layer "F.Cu") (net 41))
 (segment (start 154.41 93.9) (end 152.4 91.89) (width 0.2) (layer "F.Cu") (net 41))
 (segment (start 101.6 101.6) (end 101.6 81.28) (width 0.2) (layer "F.Cu") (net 9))
 (segment (start 101.6 81.28) (end 121.92 60.96) (width 0.2) (layer "F.Cu") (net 9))
 (segment (start 120.53 95.37) (end 120.53 64.89) (width 0.2) (layer "F.Cu") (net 10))
 (segment (start 120.53 64.89) (end 124.46 60.96) (width 0.2) (layer "F.Cu") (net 10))
 (segment (start 114.3 101.6) (end 120.53 95.37) (width 0.2) (layer "F.Cu") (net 10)))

